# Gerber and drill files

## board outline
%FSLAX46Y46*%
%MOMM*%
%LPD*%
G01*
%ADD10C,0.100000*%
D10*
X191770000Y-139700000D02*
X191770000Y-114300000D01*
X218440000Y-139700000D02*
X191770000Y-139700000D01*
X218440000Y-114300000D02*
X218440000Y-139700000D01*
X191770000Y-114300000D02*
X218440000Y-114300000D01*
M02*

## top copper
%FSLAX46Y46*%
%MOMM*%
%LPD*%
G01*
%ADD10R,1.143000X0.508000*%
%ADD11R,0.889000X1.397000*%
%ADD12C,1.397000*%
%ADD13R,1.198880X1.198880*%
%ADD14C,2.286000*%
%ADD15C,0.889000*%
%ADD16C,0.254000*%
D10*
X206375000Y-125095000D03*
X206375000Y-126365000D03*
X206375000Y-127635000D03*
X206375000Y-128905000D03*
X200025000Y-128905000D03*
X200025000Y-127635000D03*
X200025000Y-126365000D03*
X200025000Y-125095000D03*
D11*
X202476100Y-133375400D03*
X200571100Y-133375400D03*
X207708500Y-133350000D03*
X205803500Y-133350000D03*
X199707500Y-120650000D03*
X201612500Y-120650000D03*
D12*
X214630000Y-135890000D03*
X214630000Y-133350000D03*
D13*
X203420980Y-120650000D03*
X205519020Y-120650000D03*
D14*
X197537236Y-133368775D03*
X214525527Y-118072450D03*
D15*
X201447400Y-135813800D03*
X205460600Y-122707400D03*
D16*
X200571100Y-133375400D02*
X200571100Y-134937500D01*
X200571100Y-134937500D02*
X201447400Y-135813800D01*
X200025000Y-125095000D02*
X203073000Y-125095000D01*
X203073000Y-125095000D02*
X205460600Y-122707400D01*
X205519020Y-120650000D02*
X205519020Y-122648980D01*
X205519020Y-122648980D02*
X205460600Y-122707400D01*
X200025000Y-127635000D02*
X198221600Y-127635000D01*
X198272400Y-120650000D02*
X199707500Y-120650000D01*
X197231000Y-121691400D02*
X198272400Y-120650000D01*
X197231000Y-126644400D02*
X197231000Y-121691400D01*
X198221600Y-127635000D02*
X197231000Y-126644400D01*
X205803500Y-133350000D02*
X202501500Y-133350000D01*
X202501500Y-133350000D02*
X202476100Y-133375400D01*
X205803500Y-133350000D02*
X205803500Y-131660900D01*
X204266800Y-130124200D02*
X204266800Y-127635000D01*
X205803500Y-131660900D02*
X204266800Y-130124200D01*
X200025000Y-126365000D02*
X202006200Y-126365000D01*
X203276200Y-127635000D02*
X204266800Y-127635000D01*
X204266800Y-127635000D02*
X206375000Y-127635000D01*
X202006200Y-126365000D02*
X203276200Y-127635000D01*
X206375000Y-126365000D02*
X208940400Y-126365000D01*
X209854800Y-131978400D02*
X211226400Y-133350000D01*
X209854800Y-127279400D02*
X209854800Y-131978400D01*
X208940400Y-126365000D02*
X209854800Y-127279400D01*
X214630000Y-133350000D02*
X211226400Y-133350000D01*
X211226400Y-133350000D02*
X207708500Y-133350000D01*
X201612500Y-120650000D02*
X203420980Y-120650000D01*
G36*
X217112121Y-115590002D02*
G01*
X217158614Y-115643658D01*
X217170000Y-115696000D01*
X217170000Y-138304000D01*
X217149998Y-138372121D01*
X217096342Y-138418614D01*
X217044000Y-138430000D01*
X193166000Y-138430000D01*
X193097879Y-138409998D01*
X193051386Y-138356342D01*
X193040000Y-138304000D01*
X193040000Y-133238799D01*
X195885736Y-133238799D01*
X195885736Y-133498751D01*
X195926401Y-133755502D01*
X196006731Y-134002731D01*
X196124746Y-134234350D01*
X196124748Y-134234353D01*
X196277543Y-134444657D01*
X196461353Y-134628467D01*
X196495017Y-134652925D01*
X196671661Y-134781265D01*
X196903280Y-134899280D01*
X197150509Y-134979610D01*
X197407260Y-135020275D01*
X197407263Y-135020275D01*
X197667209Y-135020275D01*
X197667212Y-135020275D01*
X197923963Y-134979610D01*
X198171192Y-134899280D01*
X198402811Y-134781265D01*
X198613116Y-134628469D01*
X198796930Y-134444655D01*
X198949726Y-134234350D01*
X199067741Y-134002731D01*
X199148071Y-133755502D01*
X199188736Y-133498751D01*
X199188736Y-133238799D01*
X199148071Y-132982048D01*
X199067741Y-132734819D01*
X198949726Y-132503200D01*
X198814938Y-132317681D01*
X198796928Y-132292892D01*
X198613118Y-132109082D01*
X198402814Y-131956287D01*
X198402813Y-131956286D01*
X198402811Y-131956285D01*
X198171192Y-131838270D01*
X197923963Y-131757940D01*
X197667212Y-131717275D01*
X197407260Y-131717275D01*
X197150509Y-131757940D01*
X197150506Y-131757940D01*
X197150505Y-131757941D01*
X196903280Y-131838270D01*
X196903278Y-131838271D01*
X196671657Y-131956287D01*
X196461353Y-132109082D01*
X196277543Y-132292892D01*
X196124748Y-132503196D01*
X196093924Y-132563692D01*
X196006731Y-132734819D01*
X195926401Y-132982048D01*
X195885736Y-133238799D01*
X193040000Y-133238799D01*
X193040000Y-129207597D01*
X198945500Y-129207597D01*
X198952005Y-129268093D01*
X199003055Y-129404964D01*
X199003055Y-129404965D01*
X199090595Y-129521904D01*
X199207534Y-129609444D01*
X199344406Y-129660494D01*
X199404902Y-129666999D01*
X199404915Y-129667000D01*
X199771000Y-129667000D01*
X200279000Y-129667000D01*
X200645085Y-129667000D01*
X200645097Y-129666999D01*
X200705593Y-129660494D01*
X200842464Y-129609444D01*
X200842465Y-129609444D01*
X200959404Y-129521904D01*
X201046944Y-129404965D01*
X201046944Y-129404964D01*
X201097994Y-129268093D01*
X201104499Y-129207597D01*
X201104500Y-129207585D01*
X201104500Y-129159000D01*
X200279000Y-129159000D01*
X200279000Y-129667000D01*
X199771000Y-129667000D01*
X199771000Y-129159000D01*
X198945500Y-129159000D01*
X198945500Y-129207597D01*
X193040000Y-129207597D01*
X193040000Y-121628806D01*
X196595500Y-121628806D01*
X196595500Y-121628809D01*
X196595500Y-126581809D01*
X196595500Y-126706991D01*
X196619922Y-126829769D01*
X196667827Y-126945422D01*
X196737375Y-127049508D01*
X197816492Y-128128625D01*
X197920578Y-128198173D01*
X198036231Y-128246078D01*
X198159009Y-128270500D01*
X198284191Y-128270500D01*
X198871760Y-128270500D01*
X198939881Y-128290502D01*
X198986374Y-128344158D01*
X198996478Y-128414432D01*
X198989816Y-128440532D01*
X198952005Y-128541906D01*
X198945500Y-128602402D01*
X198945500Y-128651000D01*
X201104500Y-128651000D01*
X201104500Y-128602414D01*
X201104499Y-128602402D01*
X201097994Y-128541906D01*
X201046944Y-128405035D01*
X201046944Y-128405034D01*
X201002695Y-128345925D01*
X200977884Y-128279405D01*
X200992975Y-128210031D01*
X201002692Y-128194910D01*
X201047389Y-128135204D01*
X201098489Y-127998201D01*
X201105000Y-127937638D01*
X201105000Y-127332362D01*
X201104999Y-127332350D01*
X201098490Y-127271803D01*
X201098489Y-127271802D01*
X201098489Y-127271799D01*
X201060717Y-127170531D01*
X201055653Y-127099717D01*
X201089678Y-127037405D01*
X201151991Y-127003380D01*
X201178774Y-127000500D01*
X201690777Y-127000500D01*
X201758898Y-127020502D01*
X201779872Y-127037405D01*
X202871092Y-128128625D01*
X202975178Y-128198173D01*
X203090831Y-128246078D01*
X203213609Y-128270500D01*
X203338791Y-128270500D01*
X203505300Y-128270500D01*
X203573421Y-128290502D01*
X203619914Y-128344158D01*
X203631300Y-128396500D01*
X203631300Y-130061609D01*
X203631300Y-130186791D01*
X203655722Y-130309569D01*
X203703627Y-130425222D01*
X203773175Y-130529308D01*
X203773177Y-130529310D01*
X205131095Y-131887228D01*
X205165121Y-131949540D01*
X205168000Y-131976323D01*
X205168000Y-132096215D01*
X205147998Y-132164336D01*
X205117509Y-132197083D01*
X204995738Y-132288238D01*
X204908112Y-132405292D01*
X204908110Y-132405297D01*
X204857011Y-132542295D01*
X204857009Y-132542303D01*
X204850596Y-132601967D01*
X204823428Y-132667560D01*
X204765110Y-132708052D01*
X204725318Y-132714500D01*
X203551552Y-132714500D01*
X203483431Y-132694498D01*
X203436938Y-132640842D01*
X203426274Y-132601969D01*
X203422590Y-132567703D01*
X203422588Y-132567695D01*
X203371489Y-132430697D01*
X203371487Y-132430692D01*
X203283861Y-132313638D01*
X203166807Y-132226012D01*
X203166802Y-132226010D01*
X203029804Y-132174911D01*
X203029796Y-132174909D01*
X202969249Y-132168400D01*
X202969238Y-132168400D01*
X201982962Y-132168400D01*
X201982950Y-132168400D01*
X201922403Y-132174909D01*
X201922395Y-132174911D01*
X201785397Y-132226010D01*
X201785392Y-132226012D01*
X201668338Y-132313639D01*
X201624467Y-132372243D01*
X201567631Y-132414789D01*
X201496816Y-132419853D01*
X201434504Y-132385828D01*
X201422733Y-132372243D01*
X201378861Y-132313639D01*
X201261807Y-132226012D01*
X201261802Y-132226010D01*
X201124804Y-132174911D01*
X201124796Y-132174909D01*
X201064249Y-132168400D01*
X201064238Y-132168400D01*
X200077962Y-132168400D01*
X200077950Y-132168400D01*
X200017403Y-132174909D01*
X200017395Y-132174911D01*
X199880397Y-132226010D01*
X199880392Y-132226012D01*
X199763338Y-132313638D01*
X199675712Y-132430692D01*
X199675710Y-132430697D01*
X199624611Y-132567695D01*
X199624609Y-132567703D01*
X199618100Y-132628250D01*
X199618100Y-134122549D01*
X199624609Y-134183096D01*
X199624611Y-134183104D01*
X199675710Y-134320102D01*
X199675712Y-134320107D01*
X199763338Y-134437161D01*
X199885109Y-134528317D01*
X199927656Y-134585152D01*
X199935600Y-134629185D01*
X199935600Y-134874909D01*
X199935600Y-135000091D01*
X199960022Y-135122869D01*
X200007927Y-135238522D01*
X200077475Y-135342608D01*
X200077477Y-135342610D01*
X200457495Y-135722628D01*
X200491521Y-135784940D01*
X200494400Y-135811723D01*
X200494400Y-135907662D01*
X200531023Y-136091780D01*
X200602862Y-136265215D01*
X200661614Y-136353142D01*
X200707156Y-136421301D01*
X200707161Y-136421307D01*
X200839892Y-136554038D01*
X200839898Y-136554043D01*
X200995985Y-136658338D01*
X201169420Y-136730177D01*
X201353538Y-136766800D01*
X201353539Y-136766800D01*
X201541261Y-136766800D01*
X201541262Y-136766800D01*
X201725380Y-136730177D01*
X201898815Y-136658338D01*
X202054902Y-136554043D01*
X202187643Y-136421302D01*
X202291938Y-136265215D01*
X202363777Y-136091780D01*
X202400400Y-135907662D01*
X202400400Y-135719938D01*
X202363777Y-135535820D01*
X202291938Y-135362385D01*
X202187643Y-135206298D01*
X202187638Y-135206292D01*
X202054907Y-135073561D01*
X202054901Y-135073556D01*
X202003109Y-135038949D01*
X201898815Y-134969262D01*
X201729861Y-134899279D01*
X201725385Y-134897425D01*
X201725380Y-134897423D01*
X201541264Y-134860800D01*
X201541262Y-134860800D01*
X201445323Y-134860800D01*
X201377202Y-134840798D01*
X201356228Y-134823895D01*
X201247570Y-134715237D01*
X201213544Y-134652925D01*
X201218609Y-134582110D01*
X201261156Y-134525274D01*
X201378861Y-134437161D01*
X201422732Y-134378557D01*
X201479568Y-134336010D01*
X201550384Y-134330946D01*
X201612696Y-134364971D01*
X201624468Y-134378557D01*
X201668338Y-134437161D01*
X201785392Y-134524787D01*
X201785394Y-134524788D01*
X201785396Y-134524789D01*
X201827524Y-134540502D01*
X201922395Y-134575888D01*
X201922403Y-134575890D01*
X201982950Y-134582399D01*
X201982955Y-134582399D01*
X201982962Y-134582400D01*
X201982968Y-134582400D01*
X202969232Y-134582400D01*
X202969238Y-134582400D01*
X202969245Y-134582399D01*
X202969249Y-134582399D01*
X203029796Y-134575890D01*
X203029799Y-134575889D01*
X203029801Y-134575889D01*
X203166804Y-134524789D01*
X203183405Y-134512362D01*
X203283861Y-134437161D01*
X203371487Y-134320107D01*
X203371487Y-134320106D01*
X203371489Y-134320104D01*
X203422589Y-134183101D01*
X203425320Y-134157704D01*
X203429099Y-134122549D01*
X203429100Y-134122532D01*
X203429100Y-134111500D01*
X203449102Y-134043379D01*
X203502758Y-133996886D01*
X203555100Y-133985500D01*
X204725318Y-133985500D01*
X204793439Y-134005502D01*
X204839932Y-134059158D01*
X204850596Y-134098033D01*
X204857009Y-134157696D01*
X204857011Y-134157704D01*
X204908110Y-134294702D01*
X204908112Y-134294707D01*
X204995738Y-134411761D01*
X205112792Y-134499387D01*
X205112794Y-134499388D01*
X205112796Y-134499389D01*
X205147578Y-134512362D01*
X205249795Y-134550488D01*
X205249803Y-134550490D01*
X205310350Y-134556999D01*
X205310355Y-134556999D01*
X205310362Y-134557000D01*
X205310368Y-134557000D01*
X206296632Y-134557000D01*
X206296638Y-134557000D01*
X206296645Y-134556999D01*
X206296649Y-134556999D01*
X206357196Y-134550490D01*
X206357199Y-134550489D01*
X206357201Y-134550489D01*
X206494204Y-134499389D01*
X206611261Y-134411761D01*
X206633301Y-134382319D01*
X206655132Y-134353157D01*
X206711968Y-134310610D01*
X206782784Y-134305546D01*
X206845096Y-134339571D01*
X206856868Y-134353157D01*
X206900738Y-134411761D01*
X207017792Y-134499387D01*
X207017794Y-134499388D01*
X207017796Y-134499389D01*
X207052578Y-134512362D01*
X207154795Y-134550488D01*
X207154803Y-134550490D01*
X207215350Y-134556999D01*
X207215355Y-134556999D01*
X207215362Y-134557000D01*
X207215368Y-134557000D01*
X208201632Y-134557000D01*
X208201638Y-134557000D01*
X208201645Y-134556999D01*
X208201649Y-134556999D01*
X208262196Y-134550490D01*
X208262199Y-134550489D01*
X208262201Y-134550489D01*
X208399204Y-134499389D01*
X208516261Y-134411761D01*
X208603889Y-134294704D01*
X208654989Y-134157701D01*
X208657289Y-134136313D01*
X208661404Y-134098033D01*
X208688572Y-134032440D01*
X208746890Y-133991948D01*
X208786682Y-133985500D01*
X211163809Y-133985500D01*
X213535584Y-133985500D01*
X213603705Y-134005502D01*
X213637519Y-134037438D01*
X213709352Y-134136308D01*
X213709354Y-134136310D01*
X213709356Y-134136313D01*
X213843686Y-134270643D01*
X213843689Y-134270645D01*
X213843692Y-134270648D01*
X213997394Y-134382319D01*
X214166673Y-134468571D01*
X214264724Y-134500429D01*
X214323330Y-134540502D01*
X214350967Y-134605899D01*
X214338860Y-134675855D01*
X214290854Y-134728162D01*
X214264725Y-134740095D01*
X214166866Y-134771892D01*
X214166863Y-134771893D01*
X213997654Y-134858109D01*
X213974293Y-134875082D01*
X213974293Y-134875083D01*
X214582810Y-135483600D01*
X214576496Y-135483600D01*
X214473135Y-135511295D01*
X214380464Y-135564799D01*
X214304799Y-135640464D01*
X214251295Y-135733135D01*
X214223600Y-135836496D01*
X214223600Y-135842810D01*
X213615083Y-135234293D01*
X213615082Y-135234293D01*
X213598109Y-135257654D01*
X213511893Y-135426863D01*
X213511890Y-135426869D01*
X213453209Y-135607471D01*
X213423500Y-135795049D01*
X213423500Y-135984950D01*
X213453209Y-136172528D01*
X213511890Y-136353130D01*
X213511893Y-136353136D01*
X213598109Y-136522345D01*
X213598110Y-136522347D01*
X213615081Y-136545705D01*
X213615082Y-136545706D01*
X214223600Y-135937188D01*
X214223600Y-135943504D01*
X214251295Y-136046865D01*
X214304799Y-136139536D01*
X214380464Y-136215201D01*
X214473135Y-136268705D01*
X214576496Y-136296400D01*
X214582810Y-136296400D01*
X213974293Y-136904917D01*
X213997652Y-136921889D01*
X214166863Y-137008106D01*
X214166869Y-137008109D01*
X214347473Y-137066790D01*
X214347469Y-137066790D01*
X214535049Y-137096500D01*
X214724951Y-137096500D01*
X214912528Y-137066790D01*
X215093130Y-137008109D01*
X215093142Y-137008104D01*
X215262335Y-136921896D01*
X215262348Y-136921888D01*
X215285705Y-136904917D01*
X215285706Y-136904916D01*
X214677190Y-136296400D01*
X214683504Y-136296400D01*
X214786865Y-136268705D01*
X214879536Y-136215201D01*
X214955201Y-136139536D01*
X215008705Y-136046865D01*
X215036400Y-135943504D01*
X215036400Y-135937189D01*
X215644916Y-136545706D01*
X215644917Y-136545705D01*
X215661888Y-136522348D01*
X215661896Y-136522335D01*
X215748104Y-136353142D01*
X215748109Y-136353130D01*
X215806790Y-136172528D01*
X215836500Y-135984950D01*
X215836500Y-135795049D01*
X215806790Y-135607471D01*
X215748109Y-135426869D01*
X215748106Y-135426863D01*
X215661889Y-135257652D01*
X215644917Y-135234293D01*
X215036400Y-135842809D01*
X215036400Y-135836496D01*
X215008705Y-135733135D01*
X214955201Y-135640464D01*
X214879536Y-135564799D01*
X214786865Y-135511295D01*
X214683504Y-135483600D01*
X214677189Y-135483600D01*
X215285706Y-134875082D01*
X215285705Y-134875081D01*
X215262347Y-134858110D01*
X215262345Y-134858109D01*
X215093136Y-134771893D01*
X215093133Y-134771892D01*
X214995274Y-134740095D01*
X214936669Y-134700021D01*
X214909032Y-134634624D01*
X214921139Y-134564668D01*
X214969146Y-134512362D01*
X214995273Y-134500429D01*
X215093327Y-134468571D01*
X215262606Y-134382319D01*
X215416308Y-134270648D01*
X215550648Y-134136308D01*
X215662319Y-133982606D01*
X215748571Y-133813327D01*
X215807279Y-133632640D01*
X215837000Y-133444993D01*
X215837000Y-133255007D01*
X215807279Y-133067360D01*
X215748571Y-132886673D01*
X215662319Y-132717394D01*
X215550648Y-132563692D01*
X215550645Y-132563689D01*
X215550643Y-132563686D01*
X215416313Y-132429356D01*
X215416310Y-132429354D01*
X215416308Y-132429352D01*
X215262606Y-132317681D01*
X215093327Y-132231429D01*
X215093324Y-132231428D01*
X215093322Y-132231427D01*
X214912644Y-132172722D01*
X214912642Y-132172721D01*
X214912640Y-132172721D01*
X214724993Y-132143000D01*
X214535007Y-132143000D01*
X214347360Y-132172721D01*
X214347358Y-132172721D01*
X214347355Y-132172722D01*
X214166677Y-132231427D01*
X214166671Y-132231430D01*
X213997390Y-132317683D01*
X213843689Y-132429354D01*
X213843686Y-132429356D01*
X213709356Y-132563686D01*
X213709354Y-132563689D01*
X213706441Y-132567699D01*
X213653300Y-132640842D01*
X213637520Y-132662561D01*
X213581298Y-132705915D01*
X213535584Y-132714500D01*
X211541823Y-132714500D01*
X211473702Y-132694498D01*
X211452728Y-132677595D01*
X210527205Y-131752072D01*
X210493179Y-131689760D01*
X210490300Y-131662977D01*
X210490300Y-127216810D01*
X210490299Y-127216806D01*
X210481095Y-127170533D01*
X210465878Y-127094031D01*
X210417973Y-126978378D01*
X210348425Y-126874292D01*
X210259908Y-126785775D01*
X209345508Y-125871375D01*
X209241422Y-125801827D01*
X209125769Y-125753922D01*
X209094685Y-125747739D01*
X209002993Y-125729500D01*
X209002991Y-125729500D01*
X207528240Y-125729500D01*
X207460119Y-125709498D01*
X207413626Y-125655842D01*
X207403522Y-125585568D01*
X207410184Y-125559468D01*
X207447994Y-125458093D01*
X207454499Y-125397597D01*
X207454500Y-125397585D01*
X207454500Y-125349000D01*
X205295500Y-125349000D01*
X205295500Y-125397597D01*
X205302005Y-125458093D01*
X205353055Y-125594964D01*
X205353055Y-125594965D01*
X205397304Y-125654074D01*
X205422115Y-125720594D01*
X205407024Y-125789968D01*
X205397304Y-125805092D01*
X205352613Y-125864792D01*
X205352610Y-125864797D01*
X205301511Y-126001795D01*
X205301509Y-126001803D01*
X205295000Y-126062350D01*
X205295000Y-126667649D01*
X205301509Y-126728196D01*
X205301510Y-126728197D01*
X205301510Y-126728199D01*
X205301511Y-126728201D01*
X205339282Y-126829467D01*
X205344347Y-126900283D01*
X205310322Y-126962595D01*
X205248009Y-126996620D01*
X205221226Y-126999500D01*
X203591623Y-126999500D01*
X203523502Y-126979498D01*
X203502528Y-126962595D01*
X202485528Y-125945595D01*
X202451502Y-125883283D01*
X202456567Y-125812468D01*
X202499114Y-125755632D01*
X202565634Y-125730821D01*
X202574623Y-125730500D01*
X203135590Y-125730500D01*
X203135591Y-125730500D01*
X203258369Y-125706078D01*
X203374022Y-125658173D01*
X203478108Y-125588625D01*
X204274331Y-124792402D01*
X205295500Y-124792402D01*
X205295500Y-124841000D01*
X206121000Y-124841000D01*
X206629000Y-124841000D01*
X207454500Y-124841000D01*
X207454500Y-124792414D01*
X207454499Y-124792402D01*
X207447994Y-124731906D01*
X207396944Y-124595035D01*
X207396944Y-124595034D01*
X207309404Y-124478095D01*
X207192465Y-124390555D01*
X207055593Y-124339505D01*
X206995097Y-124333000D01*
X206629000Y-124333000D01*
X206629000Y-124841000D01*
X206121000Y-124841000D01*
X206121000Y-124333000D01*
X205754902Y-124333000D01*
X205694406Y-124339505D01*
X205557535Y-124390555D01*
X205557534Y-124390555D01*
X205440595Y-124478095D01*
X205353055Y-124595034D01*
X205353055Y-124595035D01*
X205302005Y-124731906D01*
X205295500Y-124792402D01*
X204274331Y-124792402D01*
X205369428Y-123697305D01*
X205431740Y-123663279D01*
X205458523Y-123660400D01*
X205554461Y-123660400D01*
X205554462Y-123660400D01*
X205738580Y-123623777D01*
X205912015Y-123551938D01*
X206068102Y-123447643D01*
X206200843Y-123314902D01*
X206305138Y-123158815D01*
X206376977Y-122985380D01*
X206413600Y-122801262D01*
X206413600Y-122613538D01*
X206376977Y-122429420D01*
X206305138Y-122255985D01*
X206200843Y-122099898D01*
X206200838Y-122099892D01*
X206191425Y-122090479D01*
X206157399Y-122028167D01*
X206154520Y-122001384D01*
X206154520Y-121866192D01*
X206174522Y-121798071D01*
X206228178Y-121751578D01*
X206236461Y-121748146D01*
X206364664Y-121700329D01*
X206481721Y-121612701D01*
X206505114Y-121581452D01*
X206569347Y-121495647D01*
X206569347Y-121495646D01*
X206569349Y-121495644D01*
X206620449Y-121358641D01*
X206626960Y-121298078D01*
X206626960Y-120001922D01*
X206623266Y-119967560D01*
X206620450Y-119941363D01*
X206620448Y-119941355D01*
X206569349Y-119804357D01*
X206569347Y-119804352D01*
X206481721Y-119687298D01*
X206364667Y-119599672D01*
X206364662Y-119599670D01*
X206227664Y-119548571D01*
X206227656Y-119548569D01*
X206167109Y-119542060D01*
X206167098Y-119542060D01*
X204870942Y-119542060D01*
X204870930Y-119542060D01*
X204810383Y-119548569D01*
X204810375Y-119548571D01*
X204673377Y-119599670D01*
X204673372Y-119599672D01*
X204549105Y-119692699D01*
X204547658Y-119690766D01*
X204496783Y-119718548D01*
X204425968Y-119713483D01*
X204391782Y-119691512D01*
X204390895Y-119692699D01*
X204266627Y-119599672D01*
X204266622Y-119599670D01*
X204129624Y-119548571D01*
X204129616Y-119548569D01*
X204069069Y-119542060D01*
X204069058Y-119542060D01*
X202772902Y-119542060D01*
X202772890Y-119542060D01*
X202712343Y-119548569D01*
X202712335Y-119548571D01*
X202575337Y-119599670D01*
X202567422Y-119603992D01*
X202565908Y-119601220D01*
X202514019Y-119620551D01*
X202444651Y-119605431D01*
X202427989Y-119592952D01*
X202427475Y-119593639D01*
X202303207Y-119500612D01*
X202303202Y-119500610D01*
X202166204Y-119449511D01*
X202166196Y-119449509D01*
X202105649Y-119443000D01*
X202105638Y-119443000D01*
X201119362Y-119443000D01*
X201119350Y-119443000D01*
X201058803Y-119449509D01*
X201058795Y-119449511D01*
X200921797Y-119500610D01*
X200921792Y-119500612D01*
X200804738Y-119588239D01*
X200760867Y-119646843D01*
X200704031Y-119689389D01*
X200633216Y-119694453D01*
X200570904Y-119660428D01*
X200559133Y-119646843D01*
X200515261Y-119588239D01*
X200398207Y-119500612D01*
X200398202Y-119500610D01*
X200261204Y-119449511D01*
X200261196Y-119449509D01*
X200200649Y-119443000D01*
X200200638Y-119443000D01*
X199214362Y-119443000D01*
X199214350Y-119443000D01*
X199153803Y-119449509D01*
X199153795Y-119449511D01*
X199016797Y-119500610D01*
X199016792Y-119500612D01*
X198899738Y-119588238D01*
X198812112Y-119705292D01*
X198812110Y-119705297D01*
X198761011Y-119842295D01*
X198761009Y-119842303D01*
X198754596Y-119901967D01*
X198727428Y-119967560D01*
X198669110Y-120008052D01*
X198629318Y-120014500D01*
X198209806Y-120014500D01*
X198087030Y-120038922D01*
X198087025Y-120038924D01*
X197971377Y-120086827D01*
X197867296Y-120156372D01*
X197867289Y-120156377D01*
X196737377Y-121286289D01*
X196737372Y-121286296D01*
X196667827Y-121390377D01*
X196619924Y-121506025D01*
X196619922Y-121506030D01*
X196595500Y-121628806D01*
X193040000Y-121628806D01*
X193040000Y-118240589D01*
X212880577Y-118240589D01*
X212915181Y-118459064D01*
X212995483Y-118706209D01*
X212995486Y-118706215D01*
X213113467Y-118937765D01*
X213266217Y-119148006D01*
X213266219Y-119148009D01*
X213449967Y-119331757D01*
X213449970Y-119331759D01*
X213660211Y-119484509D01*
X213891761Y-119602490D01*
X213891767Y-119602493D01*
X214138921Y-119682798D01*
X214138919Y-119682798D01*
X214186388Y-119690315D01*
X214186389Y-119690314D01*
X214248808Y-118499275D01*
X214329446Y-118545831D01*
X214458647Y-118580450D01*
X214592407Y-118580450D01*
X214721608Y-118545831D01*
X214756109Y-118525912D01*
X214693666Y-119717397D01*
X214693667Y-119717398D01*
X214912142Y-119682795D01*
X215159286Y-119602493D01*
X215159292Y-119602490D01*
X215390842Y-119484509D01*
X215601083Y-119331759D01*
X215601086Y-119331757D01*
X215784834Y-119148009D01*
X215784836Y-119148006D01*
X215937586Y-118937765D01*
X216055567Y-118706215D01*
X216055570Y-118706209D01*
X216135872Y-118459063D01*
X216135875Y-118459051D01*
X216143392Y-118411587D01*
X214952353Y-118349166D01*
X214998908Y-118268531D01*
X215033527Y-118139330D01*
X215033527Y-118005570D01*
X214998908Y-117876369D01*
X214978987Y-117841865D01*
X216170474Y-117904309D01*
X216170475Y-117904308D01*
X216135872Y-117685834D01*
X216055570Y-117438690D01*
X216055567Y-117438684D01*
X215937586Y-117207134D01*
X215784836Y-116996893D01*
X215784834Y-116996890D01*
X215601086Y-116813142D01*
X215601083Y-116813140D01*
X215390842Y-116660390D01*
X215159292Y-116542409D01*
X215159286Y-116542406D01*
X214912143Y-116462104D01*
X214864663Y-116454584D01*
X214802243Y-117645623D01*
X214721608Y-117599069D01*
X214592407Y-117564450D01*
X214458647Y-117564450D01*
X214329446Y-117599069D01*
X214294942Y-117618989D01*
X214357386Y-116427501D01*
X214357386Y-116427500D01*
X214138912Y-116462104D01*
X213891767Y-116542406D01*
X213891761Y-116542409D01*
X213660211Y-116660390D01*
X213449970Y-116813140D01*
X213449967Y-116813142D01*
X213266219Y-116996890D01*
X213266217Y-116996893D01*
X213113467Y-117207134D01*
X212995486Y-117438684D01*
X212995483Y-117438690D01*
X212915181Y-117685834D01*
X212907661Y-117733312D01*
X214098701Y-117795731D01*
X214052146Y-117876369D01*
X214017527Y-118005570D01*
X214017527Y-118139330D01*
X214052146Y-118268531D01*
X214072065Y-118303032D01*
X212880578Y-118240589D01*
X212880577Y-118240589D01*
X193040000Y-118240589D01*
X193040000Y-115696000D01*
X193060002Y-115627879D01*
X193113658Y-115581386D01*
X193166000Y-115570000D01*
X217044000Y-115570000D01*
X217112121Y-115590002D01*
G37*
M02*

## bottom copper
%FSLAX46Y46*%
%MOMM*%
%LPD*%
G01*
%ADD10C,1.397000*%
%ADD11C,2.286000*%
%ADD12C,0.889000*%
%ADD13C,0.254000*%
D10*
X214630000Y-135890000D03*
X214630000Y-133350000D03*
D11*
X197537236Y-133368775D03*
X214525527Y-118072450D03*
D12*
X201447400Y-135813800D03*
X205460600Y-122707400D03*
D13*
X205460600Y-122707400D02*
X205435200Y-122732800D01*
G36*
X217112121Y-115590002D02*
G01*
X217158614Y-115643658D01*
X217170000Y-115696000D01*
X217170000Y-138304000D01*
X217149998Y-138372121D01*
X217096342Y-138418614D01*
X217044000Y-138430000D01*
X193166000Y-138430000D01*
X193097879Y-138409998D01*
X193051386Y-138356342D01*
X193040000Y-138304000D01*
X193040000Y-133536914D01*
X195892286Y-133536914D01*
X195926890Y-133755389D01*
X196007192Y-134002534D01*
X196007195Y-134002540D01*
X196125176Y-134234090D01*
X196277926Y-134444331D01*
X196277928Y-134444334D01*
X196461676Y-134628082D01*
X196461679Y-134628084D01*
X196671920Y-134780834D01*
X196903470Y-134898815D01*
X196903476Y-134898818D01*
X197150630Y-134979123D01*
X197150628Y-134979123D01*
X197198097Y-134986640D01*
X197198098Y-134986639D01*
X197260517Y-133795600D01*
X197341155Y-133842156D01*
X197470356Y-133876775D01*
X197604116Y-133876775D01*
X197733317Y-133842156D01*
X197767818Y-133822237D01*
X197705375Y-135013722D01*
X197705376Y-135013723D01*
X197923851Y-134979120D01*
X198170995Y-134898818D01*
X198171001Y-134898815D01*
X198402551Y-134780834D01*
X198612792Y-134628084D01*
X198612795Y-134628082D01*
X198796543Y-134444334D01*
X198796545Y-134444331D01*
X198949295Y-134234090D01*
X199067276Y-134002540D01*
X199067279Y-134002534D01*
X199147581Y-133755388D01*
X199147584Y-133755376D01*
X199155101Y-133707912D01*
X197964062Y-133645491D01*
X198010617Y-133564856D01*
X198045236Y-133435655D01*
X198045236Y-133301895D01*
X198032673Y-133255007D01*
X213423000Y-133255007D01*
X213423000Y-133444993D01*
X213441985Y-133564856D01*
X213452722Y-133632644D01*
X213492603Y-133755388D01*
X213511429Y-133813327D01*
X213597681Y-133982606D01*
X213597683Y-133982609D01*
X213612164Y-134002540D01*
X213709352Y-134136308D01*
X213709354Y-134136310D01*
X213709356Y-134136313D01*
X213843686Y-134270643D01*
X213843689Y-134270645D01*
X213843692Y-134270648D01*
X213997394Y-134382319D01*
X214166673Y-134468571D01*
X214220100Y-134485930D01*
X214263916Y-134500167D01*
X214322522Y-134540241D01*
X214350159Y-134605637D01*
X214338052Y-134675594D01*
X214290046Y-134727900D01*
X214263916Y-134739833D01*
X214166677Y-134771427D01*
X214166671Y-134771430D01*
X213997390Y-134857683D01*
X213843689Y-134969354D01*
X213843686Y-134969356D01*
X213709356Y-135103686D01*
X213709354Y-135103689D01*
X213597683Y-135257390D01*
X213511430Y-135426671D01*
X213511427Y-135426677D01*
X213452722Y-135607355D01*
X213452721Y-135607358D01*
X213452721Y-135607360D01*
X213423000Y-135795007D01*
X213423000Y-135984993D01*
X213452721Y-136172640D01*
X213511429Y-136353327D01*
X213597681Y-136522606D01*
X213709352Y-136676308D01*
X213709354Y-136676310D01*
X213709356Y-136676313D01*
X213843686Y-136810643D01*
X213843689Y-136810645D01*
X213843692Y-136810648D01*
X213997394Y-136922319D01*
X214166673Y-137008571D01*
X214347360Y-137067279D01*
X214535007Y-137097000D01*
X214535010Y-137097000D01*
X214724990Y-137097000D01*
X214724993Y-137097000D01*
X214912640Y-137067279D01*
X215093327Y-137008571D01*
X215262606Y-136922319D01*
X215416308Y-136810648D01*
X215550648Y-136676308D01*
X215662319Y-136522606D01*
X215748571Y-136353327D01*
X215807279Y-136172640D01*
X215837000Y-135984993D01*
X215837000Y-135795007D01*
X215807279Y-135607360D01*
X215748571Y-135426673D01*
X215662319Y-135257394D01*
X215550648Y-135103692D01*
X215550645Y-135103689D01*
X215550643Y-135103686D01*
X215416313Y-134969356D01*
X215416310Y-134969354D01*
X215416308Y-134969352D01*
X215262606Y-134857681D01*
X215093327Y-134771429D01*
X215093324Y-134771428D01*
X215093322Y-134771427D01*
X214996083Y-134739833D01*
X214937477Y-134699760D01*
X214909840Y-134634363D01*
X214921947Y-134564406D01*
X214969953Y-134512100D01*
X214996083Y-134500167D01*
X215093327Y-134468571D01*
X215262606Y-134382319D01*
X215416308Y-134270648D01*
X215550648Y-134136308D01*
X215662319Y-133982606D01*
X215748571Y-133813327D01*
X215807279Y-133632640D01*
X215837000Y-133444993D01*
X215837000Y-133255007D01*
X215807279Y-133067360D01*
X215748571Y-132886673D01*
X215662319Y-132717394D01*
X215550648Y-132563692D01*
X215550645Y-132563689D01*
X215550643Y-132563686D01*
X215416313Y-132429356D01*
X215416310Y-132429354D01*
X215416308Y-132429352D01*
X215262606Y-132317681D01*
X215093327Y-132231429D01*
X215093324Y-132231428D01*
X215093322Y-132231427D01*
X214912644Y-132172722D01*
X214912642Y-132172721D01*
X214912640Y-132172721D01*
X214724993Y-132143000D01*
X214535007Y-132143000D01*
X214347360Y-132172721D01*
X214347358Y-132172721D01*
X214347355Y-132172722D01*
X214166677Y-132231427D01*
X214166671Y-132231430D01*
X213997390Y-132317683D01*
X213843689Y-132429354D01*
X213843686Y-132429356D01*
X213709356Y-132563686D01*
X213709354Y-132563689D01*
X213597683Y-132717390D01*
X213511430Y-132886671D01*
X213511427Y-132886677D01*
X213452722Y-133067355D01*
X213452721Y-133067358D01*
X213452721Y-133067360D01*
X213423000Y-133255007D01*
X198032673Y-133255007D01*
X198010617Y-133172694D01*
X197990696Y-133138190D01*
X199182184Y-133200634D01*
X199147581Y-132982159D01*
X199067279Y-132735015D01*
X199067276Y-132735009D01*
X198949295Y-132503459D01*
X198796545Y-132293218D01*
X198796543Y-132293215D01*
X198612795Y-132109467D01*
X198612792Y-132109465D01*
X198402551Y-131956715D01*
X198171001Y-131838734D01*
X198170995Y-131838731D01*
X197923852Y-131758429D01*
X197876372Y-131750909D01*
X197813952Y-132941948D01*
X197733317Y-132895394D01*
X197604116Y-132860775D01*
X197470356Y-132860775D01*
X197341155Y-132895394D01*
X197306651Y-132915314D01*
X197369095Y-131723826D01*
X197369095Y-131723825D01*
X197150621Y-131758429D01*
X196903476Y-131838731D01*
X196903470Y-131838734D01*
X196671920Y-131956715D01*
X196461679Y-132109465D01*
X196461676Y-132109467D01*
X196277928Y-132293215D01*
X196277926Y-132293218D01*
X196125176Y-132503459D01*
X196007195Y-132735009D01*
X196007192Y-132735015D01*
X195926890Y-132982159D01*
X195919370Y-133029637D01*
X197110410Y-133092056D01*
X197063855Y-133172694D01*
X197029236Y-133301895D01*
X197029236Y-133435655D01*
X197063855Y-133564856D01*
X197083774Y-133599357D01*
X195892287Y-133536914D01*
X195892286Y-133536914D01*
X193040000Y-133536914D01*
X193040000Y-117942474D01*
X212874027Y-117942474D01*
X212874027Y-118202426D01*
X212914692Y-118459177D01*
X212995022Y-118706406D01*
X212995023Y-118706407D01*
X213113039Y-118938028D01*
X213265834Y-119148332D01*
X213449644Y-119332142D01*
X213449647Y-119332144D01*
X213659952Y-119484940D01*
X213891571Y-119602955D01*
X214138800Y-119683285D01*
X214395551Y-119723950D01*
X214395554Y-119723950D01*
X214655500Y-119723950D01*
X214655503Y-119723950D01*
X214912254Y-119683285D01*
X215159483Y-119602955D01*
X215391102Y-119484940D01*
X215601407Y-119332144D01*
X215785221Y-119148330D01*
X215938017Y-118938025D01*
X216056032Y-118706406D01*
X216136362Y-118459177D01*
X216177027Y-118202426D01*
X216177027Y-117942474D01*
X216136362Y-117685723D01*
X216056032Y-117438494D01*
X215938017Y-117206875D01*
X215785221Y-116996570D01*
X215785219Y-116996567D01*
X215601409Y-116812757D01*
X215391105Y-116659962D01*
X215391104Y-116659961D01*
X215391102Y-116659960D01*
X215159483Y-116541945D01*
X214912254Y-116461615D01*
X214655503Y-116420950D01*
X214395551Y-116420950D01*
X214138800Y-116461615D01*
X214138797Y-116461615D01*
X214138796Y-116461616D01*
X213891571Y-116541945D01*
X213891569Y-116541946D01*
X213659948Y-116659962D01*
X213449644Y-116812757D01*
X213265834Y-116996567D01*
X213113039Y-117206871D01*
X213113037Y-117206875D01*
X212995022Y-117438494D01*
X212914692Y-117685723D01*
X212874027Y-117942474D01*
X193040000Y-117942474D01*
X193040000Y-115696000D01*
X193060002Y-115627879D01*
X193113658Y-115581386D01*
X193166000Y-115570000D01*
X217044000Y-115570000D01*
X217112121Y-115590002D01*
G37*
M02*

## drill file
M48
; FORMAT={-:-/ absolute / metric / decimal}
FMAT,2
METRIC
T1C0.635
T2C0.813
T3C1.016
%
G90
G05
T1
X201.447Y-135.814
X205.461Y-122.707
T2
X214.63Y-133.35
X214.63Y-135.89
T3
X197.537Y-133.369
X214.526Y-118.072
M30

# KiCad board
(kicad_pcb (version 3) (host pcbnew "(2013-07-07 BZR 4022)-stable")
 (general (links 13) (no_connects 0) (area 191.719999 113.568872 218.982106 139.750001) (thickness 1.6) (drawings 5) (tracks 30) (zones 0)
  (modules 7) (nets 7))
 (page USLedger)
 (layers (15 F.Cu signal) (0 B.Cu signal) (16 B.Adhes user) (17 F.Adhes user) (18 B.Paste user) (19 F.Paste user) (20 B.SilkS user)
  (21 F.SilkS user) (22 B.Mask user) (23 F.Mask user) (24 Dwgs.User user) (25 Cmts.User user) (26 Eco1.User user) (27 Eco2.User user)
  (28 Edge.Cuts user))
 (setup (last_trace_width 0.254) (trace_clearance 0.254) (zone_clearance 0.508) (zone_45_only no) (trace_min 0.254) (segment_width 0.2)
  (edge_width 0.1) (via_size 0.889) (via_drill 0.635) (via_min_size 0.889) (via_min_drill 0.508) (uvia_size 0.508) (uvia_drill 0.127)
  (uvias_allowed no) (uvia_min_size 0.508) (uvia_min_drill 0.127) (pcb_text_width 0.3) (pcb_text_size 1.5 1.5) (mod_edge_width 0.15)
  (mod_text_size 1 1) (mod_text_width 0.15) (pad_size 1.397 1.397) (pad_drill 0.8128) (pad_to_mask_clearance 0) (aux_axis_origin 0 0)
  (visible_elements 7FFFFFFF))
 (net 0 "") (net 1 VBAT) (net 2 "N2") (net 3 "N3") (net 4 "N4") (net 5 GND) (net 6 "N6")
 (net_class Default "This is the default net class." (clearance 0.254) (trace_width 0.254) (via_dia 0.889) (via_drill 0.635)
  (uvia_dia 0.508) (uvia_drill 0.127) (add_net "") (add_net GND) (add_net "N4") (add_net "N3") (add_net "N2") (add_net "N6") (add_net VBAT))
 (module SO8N (layer F.Cu) (at 203.2 127 270)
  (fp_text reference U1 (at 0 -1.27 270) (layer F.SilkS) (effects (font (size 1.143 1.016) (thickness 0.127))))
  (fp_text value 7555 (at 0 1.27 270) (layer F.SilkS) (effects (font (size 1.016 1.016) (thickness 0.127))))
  (pad 8 smd rect (at -1.905 -3.175 270) (size 0.508 1.143) (layers F.Cu F.Paste F.Mask) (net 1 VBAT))
  (pad 7 smd rect (at -0.635 -3.175 270) (size 0.508 1.143) (layers F.Cu F.Paste F.Mask) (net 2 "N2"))
  (pad 6 smd rect (at 0.635 -3.175 270) (size 0.508 1.143) (layers F.Cu F.Paste F.Mask) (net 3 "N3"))
  (pad 5 smd rect (at 1.905 -3.175 270) (size 0.508 1.143) (layers F.Cu F.Paste F.Mask))
  (pad 4 smd rect (at 1.905 3.175 270) (size 0.508 1.143) (layers F.Cu F.Paste F.Mask) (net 1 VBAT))
  (pad 3 smd rect (at 0.635 3.175 270) (size 0.508 1.143) (layers F.Cu F.Paste F.Mask) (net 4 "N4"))
  (pad 2 smd rect (at -0.635 3.175 270) (size 0.508 1.143) (layers F.Cu F.Paste F.Mask) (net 3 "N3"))
  (pad 1 smd rect (at -1.905 3.175 270) (size 0.508 1.143) (layers F.Cu F.Paste F.Mask) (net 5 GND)))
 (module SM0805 (layer F.Cu) (at 201.5236 133.3754 180)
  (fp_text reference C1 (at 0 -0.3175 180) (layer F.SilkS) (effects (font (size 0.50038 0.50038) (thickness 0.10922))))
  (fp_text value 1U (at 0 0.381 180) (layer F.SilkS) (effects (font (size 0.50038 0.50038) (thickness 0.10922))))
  (pad 1 smd rect (at -0.9525 0 180) (size 0.889 1.397) (layers F.Cu F.Paste F.Mask) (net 3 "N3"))
  (pad 2 smd rect (at 0.9525 0 180) (size 0.889 1.397) (layers F.Cu F.Paste F.Mask) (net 5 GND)))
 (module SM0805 (layer F.Cu) (at 206.756 133.35 180)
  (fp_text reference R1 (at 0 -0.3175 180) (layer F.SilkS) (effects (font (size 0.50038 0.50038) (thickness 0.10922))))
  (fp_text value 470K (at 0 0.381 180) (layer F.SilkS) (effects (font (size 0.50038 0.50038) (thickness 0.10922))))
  (pad 1 smd rect (at -0.9525 0 180) (size 0.889 1.397) (layers F.Cu F.Paste F.Mask) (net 2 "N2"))
  (pad 2 smd rect (at 0.9525 0 180) (size 0.889 1.397) (layers F.Cu F.Paste F.Mask) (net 3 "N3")))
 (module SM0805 (layer F.Cu) (at 200.66 120.65)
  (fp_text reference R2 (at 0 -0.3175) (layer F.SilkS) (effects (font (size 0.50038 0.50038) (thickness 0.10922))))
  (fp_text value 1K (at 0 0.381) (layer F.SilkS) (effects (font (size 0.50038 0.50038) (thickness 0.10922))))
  (pad 1 smd rect (at -0.9525 0) (size 0.889 1.397) (layers F.Cu F.Paste F.Mask) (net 4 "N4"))
  (pad 2 smd rect (at 0.9525 0) (size 0.889 1.397) (layers F.Cu F.Paste F.Mask) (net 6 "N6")))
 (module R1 (layer F.Cu) (at 214.63 134.62 90) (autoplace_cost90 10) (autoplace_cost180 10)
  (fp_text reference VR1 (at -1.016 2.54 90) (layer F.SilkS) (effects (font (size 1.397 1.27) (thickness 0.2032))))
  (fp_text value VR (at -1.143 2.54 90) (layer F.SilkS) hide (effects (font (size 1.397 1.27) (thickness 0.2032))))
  (pad 1 thru_hole circle (at -1.27 0 90) (size 1.397 1.397) (drill 0.8128) (layers *.Cu *.Mask F.SilkS) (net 1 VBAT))
  (pad 2 thru_hole circle (at 1.27 0 90) (size 1.397 1.397) (drill 0.8128) (layers *.Cu *.Mask F.SilkS) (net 2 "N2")))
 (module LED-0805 (layer F.Cu) (at 204.47 120.65)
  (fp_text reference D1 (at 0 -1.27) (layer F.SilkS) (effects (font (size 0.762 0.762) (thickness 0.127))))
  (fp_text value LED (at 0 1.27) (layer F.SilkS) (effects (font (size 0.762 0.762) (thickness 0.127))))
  (pad 1 smd rect (at -1.04902 0) (size 1.19888 1.19888) (layers F.Cu F.Paste F.Mask) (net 6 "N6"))
  (pad 2 smd rect (at 1.04902 0) (size 1.19888 1.19888) (layers F.Cu F.Paste F.Mask) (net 5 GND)))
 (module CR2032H (layer B.Cu) (at 203.2 128.27 42)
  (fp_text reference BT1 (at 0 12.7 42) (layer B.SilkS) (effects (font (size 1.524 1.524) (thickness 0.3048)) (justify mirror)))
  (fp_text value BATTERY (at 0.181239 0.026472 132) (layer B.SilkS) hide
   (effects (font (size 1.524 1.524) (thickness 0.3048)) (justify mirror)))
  (pad 2 thru_hole circle (at -7.62 0 42) (size 2.286 2.286) (drill 1.016) (layers *.Cu *.Mask B.SilkS) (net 5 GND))
  (pad 1 thru_hole circle (at 15.24 0 42) (size 2.286 2.286) (drill 1.016) (layers *.Cu *.Mask B.SilkS) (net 1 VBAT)))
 (gr_line (start 191.77 139.7) (end 191.77 114.3) (angle 90) (layer Edge.Cuts) (width 0.1))
 (gr_line (start 218.44 139.7) (end 191.77 139.7) (angle 90) (layer Edge.Cuts) (width 0.1))
 (gr_line (start 218.44 114.3) (end 218.44 139.7) (angle 90) (layer Edge.Cuts) (width 0.1))
 (gr_line (start 191.77 114.3) (end 218.44 114.3) (angle 90) (layer Edge.Cuts) (width 0.1))
 (segment (start 200.5711 133.3754) (end 200.5711 134.9375) (width 0.254) (layer F.Cu) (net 5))
 (via (at 201.4474 135.8138) (size 0.889) (layers F.Cu B.Cu) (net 5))
 (segment (start 200.5711 134.9375) (end 201.4474 135.8138) (width 0.254) (layer F.Cu) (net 5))
 (segment (start 200.025 125.095) (end 203.073 125.095) (width 0.254) (layer F.Cu) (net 5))
 (segment (start 203.073 125.095) (end 205.4606 122.7074) (width 0.254) (layer F.Cu) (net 5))
 (segment (start 205.51902 120.65) (end 205.51902 122.64898) (width 0.254) (layer F.Cu) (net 5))
 (segment (start 205.4606 122.7074) (end 205.4352 122.7328) (width 0.254) (layer B.Cu) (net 5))
 (via (at 205.4606 122.7074) (size 0.889) (layers F.Cu B.Cu) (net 5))
 (segment (start 205.51902 122.64898) (end 205.4606 122.7074) (width 0.254) (layer F.Cu) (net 5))
 (segment (start 200.025 127.635) (end 198.2216 127.635) (width 0.254) (layer F.Cu) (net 4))
 (segment (start 198.2724 120.65) (end 199.7075 120.65) (width 0.254) (layer F.Cu) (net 4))
 (segment (start 197.231 121.6914) (end 198.2724 120.65) (width 0.254) (layer F.Cu) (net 4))
 (segment (start 197.231 126.6444) (end 197.231 121.6914) (width 0.254) (layer F.Cu) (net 4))
 (segment (start 198.2216 127.635) (end 197.231 126.6444) (width 0.254) (layer F.Cu) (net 4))
 (segment (start 205.8035 133.35) (end 202.5015 133.35) (width 0.254) (layer F.Cu) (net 3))
 (segment (start 202.5015 133.35) (end 202.4761 133.3754) (width 0.254) (layer F.Cu) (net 3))
 (segment (start 205.8035 133.35) (end 205.8035 131.6609) (width 0.254) (layer F.Cu) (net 3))
 (segment (start 204.2668 130.1242) (end 204.2668 127.635) (width 0.254) (layer F.Cu) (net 3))
 (segment (start 205.8035 131.6609) (end 204.2668 130.1242) (width 0.254) (layer F.Cu) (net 3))
 (segment (start 200.025 126.365) (end 202.0062 126.365) (width 0.254) (layer F.Cu) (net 3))
 (segment (start 203.2762 127.635) (end 204.2668 127.635) (width 0.254) (layer F.Cu) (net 3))
 (segment (start 204.2668 127.635) (end 206.375 127.635) (width 0.254) (layer F.Cu) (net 3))
 (segment (start 202.0062 126.365) (end 203.2762 127.635) (width 0.254) (layer F.Cu) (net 3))
 (segment (start 206.375 126.365) (end 208.9404 126.365) (width 0.254) (layer F.Cu) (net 2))
 (segment (start 209.8548 131.9784) (end 211.2264 133.35) (width 0.254) (layer F.Cu) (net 2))
 (segment (start 209.8548 127.2794) (end 209.8548 131.9784) (width 0.254) (layer F.Cu) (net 2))
 (segment (start 208.9404 126.365) (end 209.8548 127.2794) (width 0.254) (layer F.Cu) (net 2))
 (segment (start 214.63 133.35) (end 211.2264 133.35) (width 0.254) (layer F.Cu) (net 2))
 (segment (start 211.2264 133.35) (end 207.7085 133.35) (width 0.254) (layer F.Cu) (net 2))
 (segment (start 201.6125 120.65) (end 203.42098 120.65) (width 0.254) (layer F.Cu) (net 6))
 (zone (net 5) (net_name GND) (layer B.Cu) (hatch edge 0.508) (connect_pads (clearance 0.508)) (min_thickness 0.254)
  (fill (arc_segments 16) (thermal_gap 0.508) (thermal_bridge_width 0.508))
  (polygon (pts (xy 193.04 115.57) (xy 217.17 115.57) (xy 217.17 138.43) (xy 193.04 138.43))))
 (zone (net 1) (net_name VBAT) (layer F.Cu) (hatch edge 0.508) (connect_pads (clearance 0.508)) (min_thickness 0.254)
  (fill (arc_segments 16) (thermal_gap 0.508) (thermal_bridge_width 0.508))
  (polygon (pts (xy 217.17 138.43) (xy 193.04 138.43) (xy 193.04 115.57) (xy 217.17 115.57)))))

